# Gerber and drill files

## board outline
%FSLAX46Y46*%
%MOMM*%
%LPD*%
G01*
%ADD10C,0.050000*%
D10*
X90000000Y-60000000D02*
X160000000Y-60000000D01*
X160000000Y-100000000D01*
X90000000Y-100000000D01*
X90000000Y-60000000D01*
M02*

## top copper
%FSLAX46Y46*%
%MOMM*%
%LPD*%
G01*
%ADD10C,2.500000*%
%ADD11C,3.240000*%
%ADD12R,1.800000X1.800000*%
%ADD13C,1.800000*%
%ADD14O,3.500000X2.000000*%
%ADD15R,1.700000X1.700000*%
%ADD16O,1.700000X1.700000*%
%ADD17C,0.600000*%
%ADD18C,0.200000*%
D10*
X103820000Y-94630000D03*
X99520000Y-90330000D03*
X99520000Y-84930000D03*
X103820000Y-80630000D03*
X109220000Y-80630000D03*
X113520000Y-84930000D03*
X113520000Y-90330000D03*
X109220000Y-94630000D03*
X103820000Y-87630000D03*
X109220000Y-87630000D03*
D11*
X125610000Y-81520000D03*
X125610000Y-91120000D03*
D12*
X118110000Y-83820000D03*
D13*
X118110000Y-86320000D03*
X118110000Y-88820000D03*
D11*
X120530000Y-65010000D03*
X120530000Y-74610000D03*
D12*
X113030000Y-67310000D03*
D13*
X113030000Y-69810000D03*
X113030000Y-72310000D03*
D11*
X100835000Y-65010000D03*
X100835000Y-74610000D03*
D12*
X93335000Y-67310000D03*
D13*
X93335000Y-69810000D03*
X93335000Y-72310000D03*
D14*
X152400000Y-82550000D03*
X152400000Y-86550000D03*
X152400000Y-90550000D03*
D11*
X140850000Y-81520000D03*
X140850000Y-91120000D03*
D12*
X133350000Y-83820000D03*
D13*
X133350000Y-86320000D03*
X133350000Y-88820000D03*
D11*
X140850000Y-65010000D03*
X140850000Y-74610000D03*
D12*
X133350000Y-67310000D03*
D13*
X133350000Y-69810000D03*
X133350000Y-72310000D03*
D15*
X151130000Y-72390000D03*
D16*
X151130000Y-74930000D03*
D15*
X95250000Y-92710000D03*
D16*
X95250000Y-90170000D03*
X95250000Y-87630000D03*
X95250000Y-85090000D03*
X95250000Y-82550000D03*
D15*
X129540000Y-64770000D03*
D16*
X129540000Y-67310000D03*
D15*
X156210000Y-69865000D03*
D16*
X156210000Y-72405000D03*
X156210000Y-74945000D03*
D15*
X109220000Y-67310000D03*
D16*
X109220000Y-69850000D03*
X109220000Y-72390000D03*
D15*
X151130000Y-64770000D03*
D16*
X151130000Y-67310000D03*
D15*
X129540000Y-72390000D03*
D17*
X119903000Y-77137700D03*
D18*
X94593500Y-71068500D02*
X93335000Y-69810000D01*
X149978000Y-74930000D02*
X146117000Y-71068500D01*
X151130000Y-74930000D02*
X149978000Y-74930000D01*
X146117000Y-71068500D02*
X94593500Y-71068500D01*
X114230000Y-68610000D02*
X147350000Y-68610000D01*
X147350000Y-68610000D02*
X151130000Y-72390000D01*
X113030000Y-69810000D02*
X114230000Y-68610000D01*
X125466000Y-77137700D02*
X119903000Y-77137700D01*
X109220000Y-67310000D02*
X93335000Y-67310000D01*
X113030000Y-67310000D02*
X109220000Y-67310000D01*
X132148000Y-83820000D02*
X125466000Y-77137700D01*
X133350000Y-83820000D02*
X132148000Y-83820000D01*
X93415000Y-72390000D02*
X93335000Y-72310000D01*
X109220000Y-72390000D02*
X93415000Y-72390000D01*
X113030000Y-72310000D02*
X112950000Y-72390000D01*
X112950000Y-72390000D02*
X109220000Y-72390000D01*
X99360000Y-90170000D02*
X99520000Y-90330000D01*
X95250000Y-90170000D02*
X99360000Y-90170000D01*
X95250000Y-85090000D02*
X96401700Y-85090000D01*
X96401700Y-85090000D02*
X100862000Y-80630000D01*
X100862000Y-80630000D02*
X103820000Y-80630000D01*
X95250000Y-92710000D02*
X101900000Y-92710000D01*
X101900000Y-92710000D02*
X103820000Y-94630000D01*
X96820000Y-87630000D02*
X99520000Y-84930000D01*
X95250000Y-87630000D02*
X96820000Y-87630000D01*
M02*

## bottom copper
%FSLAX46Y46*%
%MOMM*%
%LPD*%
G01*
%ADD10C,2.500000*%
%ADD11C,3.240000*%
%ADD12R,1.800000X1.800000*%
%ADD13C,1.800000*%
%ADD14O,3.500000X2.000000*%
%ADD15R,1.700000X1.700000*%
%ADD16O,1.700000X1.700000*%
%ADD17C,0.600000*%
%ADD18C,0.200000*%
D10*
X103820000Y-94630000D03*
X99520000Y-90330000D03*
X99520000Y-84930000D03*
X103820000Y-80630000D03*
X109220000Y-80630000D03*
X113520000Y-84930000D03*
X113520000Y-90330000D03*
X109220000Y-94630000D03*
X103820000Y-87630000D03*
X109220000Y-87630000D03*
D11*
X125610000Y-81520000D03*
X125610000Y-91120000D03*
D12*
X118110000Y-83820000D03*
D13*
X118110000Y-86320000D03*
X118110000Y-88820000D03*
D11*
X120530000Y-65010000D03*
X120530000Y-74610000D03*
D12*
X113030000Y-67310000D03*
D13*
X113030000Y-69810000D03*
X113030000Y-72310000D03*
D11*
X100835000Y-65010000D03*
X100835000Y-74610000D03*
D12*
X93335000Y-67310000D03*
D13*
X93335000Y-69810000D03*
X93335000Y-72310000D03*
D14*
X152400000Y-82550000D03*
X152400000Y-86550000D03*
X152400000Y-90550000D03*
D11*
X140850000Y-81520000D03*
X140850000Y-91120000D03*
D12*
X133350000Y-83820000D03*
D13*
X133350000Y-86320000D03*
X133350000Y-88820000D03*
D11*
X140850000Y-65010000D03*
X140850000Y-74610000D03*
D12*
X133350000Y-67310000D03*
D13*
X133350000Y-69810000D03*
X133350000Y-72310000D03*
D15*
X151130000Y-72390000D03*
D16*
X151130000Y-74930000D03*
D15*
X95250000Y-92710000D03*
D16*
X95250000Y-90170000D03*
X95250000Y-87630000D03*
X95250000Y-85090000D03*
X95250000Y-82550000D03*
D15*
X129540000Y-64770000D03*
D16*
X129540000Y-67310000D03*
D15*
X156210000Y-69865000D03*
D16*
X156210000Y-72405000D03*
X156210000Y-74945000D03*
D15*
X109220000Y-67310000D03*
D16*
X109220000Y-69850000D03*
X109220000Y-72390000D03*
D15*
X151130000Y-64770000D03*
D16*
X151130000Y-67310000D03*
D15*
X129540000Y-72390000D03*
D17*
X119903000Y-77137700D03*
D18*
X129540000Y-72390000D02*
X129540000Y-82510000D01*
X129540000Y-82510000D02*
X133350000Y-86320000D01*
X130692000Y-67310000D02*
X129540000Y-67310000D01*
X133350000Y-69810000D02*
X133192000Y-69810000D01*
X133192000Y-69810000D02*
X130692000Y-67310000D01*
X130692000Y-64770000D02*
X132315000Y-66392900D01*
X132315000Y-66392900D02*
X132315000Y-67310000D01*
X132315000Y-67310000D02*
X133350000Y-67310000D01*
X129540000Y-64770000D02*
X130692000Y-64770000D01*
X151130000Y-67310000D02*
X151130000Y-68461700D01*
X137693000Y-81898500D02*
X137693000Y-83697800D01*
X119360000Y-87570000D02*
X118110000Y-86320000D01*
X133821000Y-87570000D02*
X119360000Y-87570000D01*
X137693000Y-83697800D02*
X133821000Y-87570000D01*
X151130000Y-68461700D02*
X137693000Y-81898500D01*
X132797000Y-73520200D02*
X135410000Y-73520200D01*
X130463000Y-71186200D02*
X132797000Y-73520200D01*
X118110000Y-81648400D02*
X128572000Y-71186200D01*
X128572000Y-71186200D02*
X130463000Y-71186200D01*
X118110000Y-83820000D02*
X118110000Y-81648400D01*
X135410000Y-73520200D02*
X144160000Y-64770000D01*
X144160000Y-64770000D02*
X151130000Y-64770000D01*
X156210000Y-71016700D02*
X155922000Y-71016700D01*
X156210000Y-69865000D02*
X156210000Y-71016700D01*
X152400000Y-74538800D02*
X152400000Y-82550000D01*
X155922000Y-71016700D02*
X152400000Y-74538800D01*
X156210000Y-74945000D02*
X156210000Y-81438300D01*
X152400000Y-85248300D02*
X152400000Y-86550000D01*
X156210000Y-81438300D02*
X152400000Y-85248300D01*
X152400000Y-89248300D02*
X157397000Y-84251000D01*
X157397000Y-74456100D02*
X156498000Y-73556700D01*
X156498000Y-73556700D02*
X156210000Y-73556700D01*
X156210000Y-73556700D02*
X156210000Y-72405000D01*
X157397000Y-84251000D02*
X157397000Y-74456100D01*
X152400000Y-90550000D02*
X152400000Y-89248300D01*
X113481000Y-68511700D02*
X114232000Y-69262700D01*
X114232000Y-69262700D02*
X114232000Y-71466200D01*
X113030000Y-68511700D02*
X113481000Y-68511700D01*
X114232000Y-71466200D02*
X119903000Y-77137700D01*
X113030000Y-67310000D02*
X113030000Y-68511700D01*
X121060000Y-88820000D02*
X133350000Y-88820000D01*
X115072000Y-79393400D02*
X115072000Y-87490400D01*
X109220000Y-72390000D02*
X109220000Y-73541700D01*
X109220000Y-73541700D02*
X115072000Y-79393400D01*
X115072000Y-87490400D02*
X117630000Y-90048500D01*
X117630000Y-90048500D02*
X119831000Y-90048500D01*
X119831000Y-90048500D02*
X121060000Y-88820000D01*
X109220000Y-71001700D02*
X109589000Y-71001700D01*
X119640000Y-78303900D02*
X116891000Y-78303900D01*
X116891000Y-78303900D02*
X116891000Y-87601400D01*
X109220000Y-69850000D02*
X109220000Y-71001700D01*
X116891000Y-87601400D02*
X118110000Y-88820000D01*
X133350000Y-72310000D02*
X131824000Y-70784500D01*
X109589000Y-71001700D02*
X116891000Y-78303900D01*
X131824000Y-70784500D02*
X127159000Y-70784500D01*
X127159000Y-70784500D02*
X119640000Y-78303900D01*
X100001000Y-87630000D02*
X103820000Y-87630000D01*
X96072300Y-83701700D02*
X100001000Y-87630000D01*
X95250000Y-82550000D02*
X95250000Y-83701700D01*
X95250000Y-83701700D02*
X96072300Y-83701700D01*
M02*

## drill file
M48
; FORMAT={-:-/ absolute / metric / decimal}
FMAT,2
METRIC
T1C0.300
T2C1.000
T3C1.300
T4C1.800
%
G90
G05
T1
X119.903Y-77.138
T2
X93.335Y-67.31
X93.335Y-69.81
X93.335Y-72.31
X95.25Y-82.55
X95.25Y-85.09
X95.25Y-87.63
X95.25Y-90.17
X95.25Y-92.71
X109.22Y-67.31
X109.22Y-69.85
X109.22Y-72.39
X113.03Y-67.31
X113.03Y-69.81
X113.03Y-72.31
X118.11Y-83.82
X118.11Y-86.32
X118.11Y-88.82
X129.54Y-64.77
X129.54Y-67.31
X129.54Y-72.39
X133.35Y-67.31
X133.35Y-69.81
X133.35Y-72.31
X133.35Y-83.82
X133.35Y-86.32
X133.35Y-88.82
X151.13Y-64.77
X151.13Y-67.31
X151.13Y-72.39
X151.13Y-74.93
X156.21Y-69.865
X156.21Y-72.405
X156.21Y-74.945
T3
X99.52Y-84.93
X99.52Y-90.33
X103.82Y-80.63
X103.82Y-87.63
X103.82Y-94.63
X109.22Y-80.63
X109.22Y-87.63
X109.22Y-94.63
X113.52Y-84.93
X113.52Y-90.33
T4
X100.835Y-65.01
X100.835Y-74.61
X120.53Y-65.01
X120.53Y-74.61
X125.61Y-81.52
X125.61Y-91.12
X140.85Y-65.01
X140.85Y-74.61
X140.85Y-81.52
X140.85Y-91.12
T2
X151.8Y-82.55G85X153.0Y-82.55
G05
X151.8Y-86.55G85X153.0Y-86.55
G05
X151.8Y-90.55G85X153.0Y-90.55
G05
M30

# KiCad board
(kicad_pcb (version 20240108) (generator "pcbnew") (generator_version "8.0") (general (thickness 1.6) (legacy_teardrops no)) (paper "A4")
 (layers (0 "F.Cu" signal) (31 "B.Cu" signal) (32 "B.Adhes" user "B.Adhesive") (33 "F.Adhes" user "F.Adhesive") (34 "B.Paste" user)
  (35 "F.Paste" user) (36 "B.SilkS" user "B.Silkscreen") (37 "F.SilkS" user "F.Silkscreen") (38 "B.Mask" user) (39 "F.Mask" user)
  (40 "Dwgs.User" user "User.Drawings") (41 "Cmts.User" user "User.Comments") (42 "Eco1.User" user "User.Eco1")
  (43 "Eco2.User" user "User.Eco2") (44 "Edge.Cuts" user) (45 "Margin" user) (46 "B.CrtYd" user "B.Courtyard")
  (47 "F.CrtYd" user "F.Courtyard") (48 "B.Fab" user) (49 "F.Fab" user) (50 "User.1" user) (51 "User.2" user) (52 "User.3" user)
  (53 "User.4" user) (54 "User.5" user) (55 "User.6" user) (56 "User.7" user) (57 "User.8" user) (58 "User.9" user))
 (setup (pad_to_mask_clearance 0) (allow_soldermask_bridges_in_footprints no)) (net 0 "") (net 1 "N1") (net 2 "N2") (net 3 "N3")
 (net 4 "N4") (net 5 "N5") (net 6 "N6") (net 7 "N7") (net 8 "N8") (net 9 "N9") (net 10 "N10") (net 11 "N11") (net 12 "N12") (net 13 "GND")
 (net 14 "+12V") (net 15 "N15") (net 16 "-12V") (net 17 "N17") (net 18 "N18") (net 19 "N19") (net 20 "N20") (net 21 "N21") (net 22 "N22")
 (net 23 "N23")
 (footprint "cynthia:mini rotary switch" (layer "F.Cu") (at 106.52 87.63)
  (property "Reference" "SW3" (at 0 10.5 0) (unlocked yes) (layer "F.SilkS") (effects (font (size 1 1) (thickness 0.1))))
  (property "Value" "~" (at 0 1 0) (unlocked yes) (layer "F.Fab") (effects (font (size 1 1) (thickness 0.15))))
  (pad "1" thru_hole circle (at -2.7 7 135) (size 2.5 2.5) (drill 1.3) (layers "*.Cu" "*.Mask") (remove_unused_layers no) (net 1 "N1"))
  (pad "2" thru_hole circle (at -7 2.7 135) (size 2.5 2.5) (drill 1.3) (layers "*.Cu" "*.Mask") (remove_unused_layers no) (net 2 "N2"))
  (pad "3" thru_hole circle (at -7 -2.7 135) (size 2.5 2.5) (drill 1.3) (layers "*.Cu" "*.Mask") (remove_unused_layers no) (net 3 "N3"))
  (pad "4" thru_hole circle (at -2.7 -7 135) (size 2.5 2.5) (drill 1.3) (layers "*.Cu" "*.Mask") (remove_unused_layers no) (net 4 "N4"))
  (pad "5" thru_hole circle (at 2.7 -7 135) (size 2.5 2.5) (drill 1.3) (layers "*.Cu" "*.Mask") (remove_unused_layers no) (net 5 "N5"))
  (pad "6" thru_hole circle (at 7 -2.7 135) (size 2.5 2.5) (drill 1.3) (layers "*.Cu" "*.Mask") (remove_unused_layers no) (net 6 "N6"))
  (pad "7" thru_hole circle (at 7 2.7 135) (size 2.5 2.5) (drill 1.3) (layers "*.Cu" "*.Mask") (remove_unused_layers no) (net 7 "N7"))
  (pad "8" thru_hole circle (at 2.7 7 135) (size 2.5 2.5) (drill 1.3) (layers "*.Cu" "*.Mask") (remove_unused_layers no) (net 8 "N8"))
  (pad "9" thru_hole circle (at -2.7 0 135) (size 2.5 2.5) (drill 1.3) (layers "*.Cu" "*.Mask") (remove_unused_layers no) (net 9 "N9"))
  (pad "10" thru_hole circle (at 2.7 0 135) (size 2.5 2.5) (drill 1.3) (layers "*.Cu" "*.Mask") (remove_unused_layers no) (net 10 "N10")))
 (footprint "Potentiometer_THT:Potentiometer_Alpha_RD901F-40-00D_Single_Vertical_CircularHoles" (layer "F.Cu") (at 118.11 83.82)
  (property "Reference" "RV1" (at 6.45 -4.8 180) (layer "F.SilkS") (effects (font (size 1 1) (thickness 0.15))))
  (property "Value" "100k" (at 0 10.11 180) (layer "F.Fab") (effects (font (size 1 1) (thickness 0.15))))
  (pad "" thru_hole circle (at 7.5 -2.3 90) (size 3.24 3.24) (drill 1.8) (layers "*.Cu" "*.Mask") (remove_unused_layers no))
  (pad "" thru_hole circle (at 7.5 7.3 90) (size 3.24 3.24) (drill 1.8) (layers "*.Cu" "*.Mask") (remove_unused_layers no))
  (pad "1" thru_hole rect (at 0 0 90) (size 1.8 1.8) (drill 1) (layers "*.Cu" "*.Mask") (remove_unused_layers no) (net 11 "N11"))
  (pad "2" thru_hole circle (at 0 2.5 90) (size 1.8 1.8) (drill 1) (layers "*.Cu" "*.Mask") (remove_unused_layers no) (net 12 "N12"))
  (pad "3" thru_hole circle (at 0 5 90) (size 1.8 1.8) (drill 1) (layers "*.Cu" "*.Mask") (remove_unused_layers no) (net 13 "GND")))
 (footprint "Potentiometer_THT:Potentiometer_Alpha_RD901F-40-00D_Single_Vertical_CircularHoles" (layer "F.Cu") (at 113.03 67.31)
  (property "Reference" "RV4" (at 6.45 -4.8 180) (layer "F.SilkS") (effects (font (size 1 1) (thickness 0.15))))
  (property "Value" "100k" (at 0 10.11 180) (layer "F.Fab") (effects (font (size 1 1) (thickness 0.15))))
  (pad "" thru_hole circle (at 7.5 -2.3 90) (size 3.24 3.24) (drill 1.8) (layers "*.Cu" "*.Mask") (remove_unused_layers no))
  (pad "" thru_hole circle (at 7.5 7.3 90) (size 3.24 3.24) (drill 1.8) (layers "*.Cu" "*.Mask") (remove_unused_layers no))
  (pad "1" thru_hole rect (at 0 0 90) (size 1.8 1.8) (drill 1) (layers "*.Cu" "*.Mask") (remove_unused_layers no) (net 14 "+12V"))
  (pad "2" thru_hole circle (at 0 2.5 90) (size 1.8 1.8) (drill 1) (layers "*.Cu" "*.Mask") (remove_unused_layers no) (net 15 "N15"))
  (pad "3" thru_hole circle (at 0 5 90) (size 1.8 1.8) (drill 1) (layers "*.Cu" "*.Mask") (remove_unused_layers no) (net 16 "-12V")))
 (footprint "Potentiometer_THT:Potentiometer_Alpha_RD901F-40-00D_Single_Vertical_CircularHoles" (layer "F.Cu") (at 93.335 67.31)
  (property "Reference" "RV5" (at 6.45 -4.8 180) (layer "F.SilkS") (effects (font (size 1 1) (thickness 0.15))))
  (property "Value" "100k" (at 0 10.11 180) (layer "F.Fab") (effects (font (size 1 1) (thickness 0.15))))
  (pad "" thru_hole circle (at 7.5 -2.3 90) (size 3.24 3.24) (drill 1.8) (layers "*.Cu" "*.Mask") (remove_unused_layers no))
  (pad "" thru_hole circle (at 7.5 7.3 90) (size 3.24 3.24) (drill 1.8) (layers "*.Cu" "*.Mask") (remove_unused_layers no))
  (pad "1" thru_hole rect (at 0 0 90) (size 1.8 1.8) (drill 1) (layers "*.Cu" "*.Mask") (remove_unused_layers no) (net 14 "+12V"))
  (pad "2" thru_hole circle (at 0 2.5 90) (size 1.8 1.8) (drill 1) (layers "*.Cu" "*.Mask") (remove_unused_layers no) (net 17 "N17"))
  (pad "3" thru_hole circle (at 0 5 90) (size 1.8 1.8) (drill 1) (layers "*.Cu" "*.Mask") (remove_unused_layers no) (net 16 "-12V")))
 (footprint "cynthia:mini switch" (layer "F.Cu") (at 152.4 86.55 -90)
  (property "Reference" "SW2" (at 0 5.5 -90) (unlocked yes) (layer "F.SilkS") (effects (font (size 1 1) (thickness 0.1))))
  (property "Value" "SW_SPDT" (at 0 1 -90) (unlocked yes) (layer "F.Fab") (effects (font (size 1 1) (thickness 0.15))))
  (pad "1" thru_hole oval (at -4 0) (size 3.5 2) (drill oval 2.2 1) (layers "*.Cu" "*.Mask") (remove_unused_layers no) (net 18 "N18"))
  (pad "2" thru_hole oval (at 0 0) (size 3.5 2) (drill oval 2.2 1) (layers "*.Cu" "*.Mask") (remove_unused_layers no) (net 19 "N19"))
  (pad "3" thru_hole oval (at 4 0) (size 3.5 2) (drill oval 2.2 1) (layers "*.Cu" "*.Mask") (remove_unused_layers no) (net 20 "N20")))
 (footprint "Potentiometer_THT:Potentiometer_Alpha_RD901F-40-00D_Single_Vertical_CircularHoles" (layer "F.Cu") (at 133.35 83.82)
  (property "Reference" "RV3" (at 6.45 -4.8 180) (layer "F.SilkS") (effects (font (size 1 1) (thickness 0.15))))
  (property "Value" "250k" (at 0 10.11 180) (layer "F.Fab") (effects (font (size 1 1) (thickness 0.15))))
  (pad "" thru_hole circle (at 7.5 -2.3 90) (size 3.24 3.24) (drill 1.8) (layers "*.Cu" "*.Mask") (remove_unused_layers no))
  (pad "" thru_hole circle (at 7.5 7.3 90) (size 3.24 3.24) (drill 1.8) (layers "*.Cu" "*.Mask") (remove_unused_layers no))
  (pad "1" thru_hole rect (at 0 0 90) (size 1.8 1.8) (drill 1) (layers "*.Cu" "*.Mask") (remove_unused_layers no) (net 14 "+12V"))
  (pad "2" thru_hole circle (at 0 2.5 90) (size 1.8 1.8) (drill 1) (layers "*.Cu" "*.Mask") (remove_unused_layers no) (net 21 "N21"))
  (pad "3" thru_hole circle (at 0 5 90) (size 1.8 1.8) (drill 1) (layers "*.Cu" "*.Mask") (remove_unused_layers no) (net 16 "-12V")))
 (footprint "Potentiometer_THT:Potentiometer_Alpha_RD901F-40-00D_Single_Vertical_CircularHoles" (layer "F.Cu") (at 133.35 67.31)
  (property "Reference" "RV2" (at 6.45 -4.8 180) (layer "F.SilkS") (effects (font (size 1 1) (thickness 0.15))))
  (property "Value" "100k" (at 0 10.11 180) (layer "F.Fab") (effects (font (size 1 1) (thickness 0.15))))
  (pad "" thru_hole circle (at 7.5 -2.3 90) (size 3.24 3.24) (drill 1.8) (layers "*.Cu" "*.Mask") (remove_unused_layers no))
  (pad "" thru_hole circle (at 7.5 7.3 90) (size 3.24 3.24) (drill 1.8) (layers "*.Cu" "*.Mask") (remove_unused_layers no))
  (pad "1" thru_hole rect (at 0 0 90) (size 1.8 1.8) (drill 1) (layers "*.Cu" "*.Mask") (remove_unused_layers no) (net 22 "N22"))
  (pad "2" thru_hole circle (at 0 2.5 90) (size 1.8 1.8) (drill 1) (layers "*.Cu" "*.Mask") (remove_unused_layers no) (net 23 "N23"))
  (pad "3" thru_hole circle (at 0 5 90) (size 1.8 1.8) (drill 1) (layers "*.Cu" "*.Mask") (remove_unused_layers no) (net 13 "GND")))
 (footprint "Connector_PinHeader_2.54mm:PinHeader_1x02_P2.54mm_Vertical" (layer "B.Cu") (at 151.13 72.39 180)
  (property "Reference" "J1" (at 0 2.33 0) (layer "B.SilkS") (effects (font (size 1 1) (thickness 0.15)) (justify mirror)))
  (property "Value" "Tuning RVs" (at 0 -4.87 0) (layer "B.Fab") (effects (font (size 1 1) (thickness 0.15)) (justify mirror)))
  (pad "1" thru_hole rect (at 0 0 180) (size 1.7 1.7) (drill 1) (layers "*.Cu" "*.Mask") (remove_unused_layers no) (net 15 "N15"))
  (pad "2" thru_hole oval (at 0 -2.54 180) (size 1.7 1.7) (drill 1) (layers "*.Cu" "*.Mask") (remove_unused_layers no) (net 17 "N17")))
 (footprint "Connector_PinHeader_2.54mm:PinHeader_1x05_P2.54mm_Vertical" (layer "B.Cu") (at 95.25 92.71)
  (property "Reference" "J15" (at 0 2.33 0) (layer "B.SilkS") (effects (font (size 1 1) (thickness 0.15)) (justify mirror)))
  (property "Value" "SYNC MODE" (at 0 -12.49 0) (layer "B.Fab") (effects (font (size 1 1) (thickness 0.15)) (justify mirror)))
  (pad "1" thru_hole rect (at 0 0) (size 1.7 1.7) (drill 1) (layers "*.Cu" "*.Mask") (remove_unused_layers no) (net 1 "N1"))
  (pad "2" thru_hole oval (at 0 -2.54) (size 1.7 1.7) (drill 1) (layers "*.Cu" "*.Mask") (remove_unused_layers no) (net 2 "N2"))
  (pad "3" thru_hole oval (at 0 -5.08) (size 1.7 1.7) (drill 1) (layers "*.Cu" "*.Mask") (remove_unused_layers no) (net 3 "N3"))
  (pad "4" thru_hole oval (at 0 -7.62) (size 1.7 1.7) (drill 1) (layers "*.Cu" "*.Mask") (remove_unused_layers no) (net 4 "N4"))
  (pad "5" thru_hole oval (at 0 -10.16) (size 1.7 1.7) (drill 1) (layers "*.Cu" "*.Mask") (remove_unused_layers no) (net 9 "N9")))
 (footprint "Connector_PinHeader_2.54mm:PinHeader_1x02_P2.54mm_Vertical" (layer "B.Cu") (at 129.54 64.77 180)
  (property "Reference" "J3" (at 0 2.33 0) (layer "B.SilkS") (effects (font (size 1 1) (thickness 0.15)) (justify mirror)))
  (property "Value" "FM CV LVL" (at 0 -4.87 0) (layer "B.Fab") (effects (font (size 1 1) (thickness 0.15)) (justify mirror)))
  (pad "1" thru_hole rect (at 0 0 180) (size 1.7 1.7) (drill 1) (layers "*.Cu" "*.Mask") (remove_unused_layers no) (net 22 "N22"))
  (pad "2" thru_hole oval (at 0 -2.54 180) (size 1.7 1.7) (drill 1) (layers "*.Cu" "*.Mask") (remove_unused_layers no) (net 23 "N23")))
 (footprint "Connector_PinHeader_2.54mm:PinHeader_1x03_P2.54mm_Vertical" (layer "B.Cu") (at 156.21 69.865 180)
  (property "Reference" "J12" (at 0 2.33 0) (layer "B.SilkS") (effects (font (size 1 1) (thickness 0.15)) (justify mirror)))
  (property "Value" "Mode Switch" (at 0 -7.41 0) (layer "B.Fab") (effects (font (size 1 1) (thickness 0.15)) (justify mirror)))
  (pad "1" thru_hole rect (at 0 0 180) (size 1.7 1.7) (drill 1) (layers "*.Cu" "*.Mask") (remove_unused_layers no) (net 18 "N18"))
  (pad "2" thru_hole oval (at 0 -2.54 180) (size 1.7 1.7) (drill 1) (layers "*.Cu" "*.Mask") (remove_unused_layers no) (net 20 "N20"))
  (pad "3" thru_hole oval (at 0 -5.08 180) (size 1.7 1.7) (drill 1) (layers "*.Cu" "*.Mask") (remove_unused_layers no) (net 19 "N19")))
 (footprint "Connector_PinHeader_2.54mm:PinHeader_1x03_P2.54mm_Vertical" (layer "B.Cu") (at 109.22 67.31 180)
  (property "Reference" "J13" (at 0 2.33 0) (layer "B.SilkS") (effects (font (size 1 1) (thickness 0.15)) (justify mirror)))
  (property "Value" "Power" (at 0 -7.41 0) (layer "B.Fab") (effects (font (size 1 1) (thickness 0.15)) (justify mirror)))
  (pad "1" thru_hole rect (at 0 0 180) (size 1.7 1.7) (drill 1) (layers "*.Cu" "*.Mask") (remove_unused_layers no) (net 14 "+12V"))
  (pad "2" thru_hole oval (at 0 -2.54 180) (size 1.7 1.7) (drill 1) (layers "*.Cu" "*.Mask") (remove_unused_layers no) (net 13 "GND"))
  (pad "3" thru_hole oval (at 0 -5.08 180) (size 1.7 1.7) (drill 1) (layers "*.Cu" "*.Mask") (remove_unused_layers no) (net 16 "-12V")))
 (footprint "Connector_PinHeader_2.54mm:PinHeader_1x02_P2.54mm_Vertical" (layer "B.Cu") (at 151.13 64.77 180)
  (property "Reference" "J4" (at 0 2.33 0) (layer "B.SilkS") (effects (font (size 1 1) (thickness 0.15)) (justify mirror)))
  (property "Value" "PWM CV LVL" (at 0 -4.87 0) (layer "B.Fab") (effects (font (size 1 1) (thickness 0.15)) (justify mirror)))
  (pad "1" thru_hole rect (at 0 0 180) (size 1.7 1.7) (drill 1) (layers "*.Cu" "*.Mask") (remove_unused_layers no) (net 11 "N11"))
  (pad "2" thru_hole oval (at 0 -2.54 180) (size 1.7 1.7) (drill 1) (layers "*.Cu" "*.Mask") (remove_unused_layers no) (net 12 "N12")))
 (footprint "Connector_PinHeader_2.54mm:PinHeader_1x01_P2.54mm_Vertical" (layer "B.Cu") (at 129.54 72.39 180)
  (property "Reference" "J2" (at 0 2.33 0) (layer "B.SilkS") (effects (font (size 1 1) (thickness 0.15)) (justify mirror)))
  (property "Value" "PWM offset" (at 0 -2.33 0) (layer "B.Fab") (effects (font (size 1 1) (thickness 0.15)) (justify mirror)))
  (pad "1" thru_hole rect (at 0 0 180) (size 1.7 1.7) (drill 1) (layers "*.Cu" "*.Mask") (remove_unused_layers no) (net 21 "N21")))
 (gr_rect (start 90 60) (end 160 100) (stroke (width 0.05) (type default)) (fill none) (layer "Edge.Cuts"))
 (segment (start 94.5935 71.0685) (end 93.335 69.81) (width 0.2) (layer "F.Cu") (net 17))
 (segment (start 149.978 74.93) (end 146.117 71.0685) (width 0.2) (layer "F.Cu") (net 17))
 (segment (start 151.13 74.93) (end 149.978 74.93) (width 0.2) (layer "F.Cu") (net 17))
 (segment (start 146.117 71.0685) (end 94.5935 71.0685) (width 0.2) (layer "F.Cu") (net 17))
 (segment (start 114.23 68.61) (end 147.35 68.61) (width 0.2) (layer "F.Cu") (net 15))
 (segment (start 147.35 68.61) (end 151.13 72.39) (width 0.2) (layer "F.Cu") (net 15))
 (segment (start 113.03 69.81) (end 114.23 68.61) (width 0.2) (layer "F.Cu") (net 15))
 (segment (start 129.54 72.39) (end 129.54 82.51) (width 0.2) (layer "B.Cu") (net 21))
 (segment (start 129.54 82.51) (end 133.35 86.32) (width 0.2) (layer "B.Cu") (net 21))
 (segment (start 130.692 67.31) (end 129.54 67.31) (width 0.2) (layer "B.Cu") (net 23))
 (segment (start 133.35 69.81) (end 133.192 69.81) (width 0.2) (layer "B.Cu") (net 23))
 (segment (start 133.192 69.81) (end 130.692 67.31) (width 0.2) (layer "B.Cu") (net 23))
 (segment (start 130.692 64.77) (end 132.315 66.3929) (width 0.2) (layer "B.Cu") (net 22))
 (segment (start 132.315 66.3929) (end 132.315 67.31) (width 0.2) (layer "B.Cu") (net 22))
 (segment (start 132.315 67.31) (end 133.35 67.31) (width 0.2) (layer "B.Cu") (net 22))
 (segment (start 129.54 64.77) (end 130.692 64.77) (width 0.2) (layer "B.Cu") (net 22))
 (segment (start 151.13 67.31) (end 151.13 68.4617) (width 0.2) (layer "B.Cu") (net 12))
 (segment (start 137.693 81.8985) (end 137.693 83.6978) (width 0.2) (layer "B.Cu") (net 12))
 (segment (start 119.36 87.57) (end 118.11 86.32) (width 0.2) (layer "B.Cu") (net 12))
 (segment (start 133.821 87.57) (end 119.36 87.57) (width 0.2) (layer "B.Cu") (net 12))
 (segment (start 137.693 83.6978) (end 133.821 87.57) (width 0.2) (layer "B.Cu") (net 12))
 (segment (start 151.13 68.4617) (end 137.693 81.8985) (width 0.2) (layer "B.Cu") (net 12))
 (segment (start 132.797 73.5202) (end 135.41 73.5202) (width 0.2) (layer "B.Cu") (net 11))
 (segment (start 130.463 71.1862) (end 132.797 73.5202) (width 0.2) (layer "B.Cu") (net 11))
 (segment (start 118.11 81.6484) (end 128.572 71.1862) (width 0.2) (layer "B.Cu") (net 11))
 (segment (start 128.572 71.1862) (end 130.463 71.1862) (width 0.2) (layer "B.Cu") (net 11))
 (segment (start 118.11 83.82) (end 118.11 81.6484) (width 0.2) (layer "B.Cu") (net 11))
 (segment (start 135.41 73.5202) (end 144.16 64.77) (width 0.2) (layer "B.Cu") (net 11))
 (segment (start 144.16 64.77) (end 151.13 64.77) (width 0.2) (layer "B.Cu") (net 11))
 (segment (start 156.21 71.0167) (end 155.922 71.0167) (width 0.2) (layer "B.Cu") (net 18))
 (segment (start 156.21 69.865) (end 156.21 71.0167) (width 0.2) (layer "B.Cu") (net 18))
 (segment (start 152.4 74.5388) (end 152.4 82.55) (width 0.2) (layer "B.Cu") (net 18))
 (segment (start 155.922 71.0167) (end 152.4 74.5388) (width 0.2) (layer "B.Cu") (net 18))
 (segment (start 156.21 74.945) (end 156.21 81.4383) (width 0.2) (layer "B.Cu") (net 19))
 (segment (start 152.4 85.2483) (end 152.4 86.55) (width 0.2) (layer "B.Cu") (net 19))
 (segment (start 156.21 81.4383) (end 152.4 85.2483) (width 0.2) (layer "B.Cu") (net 19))
 (segment (start 152.4 89.2483) (end 157.397 84.251) (width 0.2) (layer "B.Cu") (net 20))
 (segment (start 157.397 74.4561) (end 156.498 73.5567) (width 0.2) (layer "B.Cu") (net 20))
 (segment (start 156.498 73.5567) (end 156.21 73.5567) (width 0.2) (layer "B.Cu") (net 20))
 (segment (start 156.21 73.5567) (end 156.21 72.405) (width 0.2) (layer "B.Cu") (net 20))
 (segment (start 157.397 84.251) (end 157.397 74.4561) (width 0.2) (layer "B.Cu") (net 20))
 (segment (start 152.4 90.55) (end 152.4 89.2483) (width 0.2) (layer "B.Cu") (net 20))
 (segment (start 125.466 77.1377) (end 119.903 77.1377) (width 0.2) (layer "F.Cu") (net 14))
 (segment (start 109.22 67.31) (end 93.335 67.31) (width 0.2) (layer "F.Cu") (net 14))
 (segment (start 113.03 67.31) (end 109.22 67.31) (width 0.2) (layer "F.Cu") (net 14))
 (segment (start 132.148 83.82) (end 125.466 77.1377) (width 0.2) (layer "F.Cu") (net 14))
 (segment (start 133.35 83.82) (end 132.148 83.82) (width 0.2) (layer "F.Cu") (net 14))
 (via (at 119.903 77.1377) (size 0.6) (drill 0.3) (layers "F.Cu" "B.Cu") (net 14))
 (segment (start 113.481 68.5117) (end 114.232 69.2627) (width 0.2) (layer "B.Cu") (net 14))
 (segment (start 114.232 69.2627) (end 114.232 71.4662) (width 0.2) (layer "B.Cu") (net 14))
 (segment (start 113.03 68.5117) (end 113.481 68.5117) (width 0.2) (layer "B.Cu") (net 14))
 (segment (start 114.232 71.4662) (end 119.903 77.1377) (width 0.2) (layer "B.Cu") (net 14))
 (segment (start 113.03 67.31) (end 113.03 68.5117) (width 0.2) (layer "B.Cu") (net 14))
 (segment (start 93.415 72.39) (end 93.335 72.31) (width 0.2) (layer "F.Cu") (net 16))
 (segment (start 109.22 72.39) (end 93.415 72.39) (width 0.2) (layer "F.Cu") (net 16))
 (segment (start 113.03 72.31) (end 112.95 72.39) (width 0.2) (layer "F.Cu") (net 16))
 (segment (start 112.95 72.39) (end 109.22 72.39) (width 0.2) (layer "F.Cu") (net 16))
 (segment (start 121.06 88.82) (end 133.35 88.82) (width 0.2) (layer "B.Cu") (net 16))
 (segment (start 115.072 79.3934) (end 115.072 87.4904) (width 0.2) (layer "B.Cu") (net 16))
 (segment (start 109.22 72.39) (end 109.22 73.5417) (width 0.2) (layer "B.Cu") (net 16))
 (segment (start 109.22 73.5417) (end 115.072 79.3934) (width 0.2) (layer "B.Cu") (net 16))
 (segment (start 115.072 87.4904) (end 117.63 90.0485) (width 0.2) (layer "B.Cu") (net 16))
 (segment (start 117.63 90.0485) (end 119.831 90.0485) (width 0.2) (layer "B.Cu") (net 16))
 (segment (start 119.831 90.0485) (end 121.06 88.82) (width 0.2) (layer "B.Cu") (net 16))
 (segment (start 109.22 71.0017) (end 109.589 71.0017) (width 0.2) (layer "B.Cu") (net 13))
 (segment (start 119.64 78.3039) (end 116.891 78.3039) (width 0.2) (layer "B.Cu") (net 13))
 (segment (start 116.891 78.3039) (end 116.891 87.6014) (width 0.2) (layer "B.Cu") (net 13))
 (segment (start 109.22 69.85) (end 109.22 71.0017) (width 0.2) (layer "B.Cu") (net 13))
 (segment (start 116.891 87.6014) (end 118.11 88.82) (width 0.2) (layer "B.Cu") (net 13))
 (segment (start 133.35 72.31) (end 131.824 70.7845) (width 0.2) (layer "B.Cu") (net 13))
 (segment (start 109.589 71.0017) (end 116.891 78.3039) (width 0.2) (layer "B.Cu") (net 13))
 (segment (start 131.824 70.7845) (end 127.159 70.7845) (width 0.2) (layer "B.Cu") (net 13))
 (segment (start 127.159 70.7845) (end 119.64 78.3039) (width 0.2) (layer "B.Cu") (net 13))
 (segment (start 99.36 90.17) (end 99.52 90.33) (width 0.2) (layer "F.Cu") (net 2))
 (segment (start 95.25 90.17) (end 99.36 90.17) (width 0.2) (layer "F.Cu") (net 2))
 (segment (start 95.25 85.09) (end 96.4017 85.09) (width 0.2) (layer "F.Cu") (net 4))
 (segment (start 96.4017 85.09) (end 100.862 80.63) (width 0.2) (layer "F.Cu") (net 4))
 (segment (start 100.862 80.63) (end 103.82 80.63) (width 0.2) (layer "F.Cu") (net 4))
 (segment (start 100.001 87.63) (end 103.82 87.63) (width 0.2) (layer "B.Cu") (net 9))
 (segment (start 96.0723 83.7017) (end 100.001 87.63) (width 0.2) (layer "B.Cu") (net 9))
 (segment (start 95.25 82.55) (end 95.25 83.7017) (width 0.2) (layer "B.Cu") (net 9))
 (segment (start 95.25 83.7017) (end 96.0723 83.7017) (width 0.2) (layer "B.Cu") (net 9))
 (segment (start 95.25 92.71) (end 101.9 92.71) (width 0.2) (layer "F.Cu") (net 1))
 (segment (start 101.9 92.71) (end 103.82 94.63) (width 0.2) (layer "F.Cu") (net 1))
 (segment (start 96.82 87.63) (end 99.52 84.93) (width 0.2) (layer "F.Cu") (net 3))
 (segment (start 95.25 87.63) (end 96.82 87.63) (width 0.2) (layer "F.Cu") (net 3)))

